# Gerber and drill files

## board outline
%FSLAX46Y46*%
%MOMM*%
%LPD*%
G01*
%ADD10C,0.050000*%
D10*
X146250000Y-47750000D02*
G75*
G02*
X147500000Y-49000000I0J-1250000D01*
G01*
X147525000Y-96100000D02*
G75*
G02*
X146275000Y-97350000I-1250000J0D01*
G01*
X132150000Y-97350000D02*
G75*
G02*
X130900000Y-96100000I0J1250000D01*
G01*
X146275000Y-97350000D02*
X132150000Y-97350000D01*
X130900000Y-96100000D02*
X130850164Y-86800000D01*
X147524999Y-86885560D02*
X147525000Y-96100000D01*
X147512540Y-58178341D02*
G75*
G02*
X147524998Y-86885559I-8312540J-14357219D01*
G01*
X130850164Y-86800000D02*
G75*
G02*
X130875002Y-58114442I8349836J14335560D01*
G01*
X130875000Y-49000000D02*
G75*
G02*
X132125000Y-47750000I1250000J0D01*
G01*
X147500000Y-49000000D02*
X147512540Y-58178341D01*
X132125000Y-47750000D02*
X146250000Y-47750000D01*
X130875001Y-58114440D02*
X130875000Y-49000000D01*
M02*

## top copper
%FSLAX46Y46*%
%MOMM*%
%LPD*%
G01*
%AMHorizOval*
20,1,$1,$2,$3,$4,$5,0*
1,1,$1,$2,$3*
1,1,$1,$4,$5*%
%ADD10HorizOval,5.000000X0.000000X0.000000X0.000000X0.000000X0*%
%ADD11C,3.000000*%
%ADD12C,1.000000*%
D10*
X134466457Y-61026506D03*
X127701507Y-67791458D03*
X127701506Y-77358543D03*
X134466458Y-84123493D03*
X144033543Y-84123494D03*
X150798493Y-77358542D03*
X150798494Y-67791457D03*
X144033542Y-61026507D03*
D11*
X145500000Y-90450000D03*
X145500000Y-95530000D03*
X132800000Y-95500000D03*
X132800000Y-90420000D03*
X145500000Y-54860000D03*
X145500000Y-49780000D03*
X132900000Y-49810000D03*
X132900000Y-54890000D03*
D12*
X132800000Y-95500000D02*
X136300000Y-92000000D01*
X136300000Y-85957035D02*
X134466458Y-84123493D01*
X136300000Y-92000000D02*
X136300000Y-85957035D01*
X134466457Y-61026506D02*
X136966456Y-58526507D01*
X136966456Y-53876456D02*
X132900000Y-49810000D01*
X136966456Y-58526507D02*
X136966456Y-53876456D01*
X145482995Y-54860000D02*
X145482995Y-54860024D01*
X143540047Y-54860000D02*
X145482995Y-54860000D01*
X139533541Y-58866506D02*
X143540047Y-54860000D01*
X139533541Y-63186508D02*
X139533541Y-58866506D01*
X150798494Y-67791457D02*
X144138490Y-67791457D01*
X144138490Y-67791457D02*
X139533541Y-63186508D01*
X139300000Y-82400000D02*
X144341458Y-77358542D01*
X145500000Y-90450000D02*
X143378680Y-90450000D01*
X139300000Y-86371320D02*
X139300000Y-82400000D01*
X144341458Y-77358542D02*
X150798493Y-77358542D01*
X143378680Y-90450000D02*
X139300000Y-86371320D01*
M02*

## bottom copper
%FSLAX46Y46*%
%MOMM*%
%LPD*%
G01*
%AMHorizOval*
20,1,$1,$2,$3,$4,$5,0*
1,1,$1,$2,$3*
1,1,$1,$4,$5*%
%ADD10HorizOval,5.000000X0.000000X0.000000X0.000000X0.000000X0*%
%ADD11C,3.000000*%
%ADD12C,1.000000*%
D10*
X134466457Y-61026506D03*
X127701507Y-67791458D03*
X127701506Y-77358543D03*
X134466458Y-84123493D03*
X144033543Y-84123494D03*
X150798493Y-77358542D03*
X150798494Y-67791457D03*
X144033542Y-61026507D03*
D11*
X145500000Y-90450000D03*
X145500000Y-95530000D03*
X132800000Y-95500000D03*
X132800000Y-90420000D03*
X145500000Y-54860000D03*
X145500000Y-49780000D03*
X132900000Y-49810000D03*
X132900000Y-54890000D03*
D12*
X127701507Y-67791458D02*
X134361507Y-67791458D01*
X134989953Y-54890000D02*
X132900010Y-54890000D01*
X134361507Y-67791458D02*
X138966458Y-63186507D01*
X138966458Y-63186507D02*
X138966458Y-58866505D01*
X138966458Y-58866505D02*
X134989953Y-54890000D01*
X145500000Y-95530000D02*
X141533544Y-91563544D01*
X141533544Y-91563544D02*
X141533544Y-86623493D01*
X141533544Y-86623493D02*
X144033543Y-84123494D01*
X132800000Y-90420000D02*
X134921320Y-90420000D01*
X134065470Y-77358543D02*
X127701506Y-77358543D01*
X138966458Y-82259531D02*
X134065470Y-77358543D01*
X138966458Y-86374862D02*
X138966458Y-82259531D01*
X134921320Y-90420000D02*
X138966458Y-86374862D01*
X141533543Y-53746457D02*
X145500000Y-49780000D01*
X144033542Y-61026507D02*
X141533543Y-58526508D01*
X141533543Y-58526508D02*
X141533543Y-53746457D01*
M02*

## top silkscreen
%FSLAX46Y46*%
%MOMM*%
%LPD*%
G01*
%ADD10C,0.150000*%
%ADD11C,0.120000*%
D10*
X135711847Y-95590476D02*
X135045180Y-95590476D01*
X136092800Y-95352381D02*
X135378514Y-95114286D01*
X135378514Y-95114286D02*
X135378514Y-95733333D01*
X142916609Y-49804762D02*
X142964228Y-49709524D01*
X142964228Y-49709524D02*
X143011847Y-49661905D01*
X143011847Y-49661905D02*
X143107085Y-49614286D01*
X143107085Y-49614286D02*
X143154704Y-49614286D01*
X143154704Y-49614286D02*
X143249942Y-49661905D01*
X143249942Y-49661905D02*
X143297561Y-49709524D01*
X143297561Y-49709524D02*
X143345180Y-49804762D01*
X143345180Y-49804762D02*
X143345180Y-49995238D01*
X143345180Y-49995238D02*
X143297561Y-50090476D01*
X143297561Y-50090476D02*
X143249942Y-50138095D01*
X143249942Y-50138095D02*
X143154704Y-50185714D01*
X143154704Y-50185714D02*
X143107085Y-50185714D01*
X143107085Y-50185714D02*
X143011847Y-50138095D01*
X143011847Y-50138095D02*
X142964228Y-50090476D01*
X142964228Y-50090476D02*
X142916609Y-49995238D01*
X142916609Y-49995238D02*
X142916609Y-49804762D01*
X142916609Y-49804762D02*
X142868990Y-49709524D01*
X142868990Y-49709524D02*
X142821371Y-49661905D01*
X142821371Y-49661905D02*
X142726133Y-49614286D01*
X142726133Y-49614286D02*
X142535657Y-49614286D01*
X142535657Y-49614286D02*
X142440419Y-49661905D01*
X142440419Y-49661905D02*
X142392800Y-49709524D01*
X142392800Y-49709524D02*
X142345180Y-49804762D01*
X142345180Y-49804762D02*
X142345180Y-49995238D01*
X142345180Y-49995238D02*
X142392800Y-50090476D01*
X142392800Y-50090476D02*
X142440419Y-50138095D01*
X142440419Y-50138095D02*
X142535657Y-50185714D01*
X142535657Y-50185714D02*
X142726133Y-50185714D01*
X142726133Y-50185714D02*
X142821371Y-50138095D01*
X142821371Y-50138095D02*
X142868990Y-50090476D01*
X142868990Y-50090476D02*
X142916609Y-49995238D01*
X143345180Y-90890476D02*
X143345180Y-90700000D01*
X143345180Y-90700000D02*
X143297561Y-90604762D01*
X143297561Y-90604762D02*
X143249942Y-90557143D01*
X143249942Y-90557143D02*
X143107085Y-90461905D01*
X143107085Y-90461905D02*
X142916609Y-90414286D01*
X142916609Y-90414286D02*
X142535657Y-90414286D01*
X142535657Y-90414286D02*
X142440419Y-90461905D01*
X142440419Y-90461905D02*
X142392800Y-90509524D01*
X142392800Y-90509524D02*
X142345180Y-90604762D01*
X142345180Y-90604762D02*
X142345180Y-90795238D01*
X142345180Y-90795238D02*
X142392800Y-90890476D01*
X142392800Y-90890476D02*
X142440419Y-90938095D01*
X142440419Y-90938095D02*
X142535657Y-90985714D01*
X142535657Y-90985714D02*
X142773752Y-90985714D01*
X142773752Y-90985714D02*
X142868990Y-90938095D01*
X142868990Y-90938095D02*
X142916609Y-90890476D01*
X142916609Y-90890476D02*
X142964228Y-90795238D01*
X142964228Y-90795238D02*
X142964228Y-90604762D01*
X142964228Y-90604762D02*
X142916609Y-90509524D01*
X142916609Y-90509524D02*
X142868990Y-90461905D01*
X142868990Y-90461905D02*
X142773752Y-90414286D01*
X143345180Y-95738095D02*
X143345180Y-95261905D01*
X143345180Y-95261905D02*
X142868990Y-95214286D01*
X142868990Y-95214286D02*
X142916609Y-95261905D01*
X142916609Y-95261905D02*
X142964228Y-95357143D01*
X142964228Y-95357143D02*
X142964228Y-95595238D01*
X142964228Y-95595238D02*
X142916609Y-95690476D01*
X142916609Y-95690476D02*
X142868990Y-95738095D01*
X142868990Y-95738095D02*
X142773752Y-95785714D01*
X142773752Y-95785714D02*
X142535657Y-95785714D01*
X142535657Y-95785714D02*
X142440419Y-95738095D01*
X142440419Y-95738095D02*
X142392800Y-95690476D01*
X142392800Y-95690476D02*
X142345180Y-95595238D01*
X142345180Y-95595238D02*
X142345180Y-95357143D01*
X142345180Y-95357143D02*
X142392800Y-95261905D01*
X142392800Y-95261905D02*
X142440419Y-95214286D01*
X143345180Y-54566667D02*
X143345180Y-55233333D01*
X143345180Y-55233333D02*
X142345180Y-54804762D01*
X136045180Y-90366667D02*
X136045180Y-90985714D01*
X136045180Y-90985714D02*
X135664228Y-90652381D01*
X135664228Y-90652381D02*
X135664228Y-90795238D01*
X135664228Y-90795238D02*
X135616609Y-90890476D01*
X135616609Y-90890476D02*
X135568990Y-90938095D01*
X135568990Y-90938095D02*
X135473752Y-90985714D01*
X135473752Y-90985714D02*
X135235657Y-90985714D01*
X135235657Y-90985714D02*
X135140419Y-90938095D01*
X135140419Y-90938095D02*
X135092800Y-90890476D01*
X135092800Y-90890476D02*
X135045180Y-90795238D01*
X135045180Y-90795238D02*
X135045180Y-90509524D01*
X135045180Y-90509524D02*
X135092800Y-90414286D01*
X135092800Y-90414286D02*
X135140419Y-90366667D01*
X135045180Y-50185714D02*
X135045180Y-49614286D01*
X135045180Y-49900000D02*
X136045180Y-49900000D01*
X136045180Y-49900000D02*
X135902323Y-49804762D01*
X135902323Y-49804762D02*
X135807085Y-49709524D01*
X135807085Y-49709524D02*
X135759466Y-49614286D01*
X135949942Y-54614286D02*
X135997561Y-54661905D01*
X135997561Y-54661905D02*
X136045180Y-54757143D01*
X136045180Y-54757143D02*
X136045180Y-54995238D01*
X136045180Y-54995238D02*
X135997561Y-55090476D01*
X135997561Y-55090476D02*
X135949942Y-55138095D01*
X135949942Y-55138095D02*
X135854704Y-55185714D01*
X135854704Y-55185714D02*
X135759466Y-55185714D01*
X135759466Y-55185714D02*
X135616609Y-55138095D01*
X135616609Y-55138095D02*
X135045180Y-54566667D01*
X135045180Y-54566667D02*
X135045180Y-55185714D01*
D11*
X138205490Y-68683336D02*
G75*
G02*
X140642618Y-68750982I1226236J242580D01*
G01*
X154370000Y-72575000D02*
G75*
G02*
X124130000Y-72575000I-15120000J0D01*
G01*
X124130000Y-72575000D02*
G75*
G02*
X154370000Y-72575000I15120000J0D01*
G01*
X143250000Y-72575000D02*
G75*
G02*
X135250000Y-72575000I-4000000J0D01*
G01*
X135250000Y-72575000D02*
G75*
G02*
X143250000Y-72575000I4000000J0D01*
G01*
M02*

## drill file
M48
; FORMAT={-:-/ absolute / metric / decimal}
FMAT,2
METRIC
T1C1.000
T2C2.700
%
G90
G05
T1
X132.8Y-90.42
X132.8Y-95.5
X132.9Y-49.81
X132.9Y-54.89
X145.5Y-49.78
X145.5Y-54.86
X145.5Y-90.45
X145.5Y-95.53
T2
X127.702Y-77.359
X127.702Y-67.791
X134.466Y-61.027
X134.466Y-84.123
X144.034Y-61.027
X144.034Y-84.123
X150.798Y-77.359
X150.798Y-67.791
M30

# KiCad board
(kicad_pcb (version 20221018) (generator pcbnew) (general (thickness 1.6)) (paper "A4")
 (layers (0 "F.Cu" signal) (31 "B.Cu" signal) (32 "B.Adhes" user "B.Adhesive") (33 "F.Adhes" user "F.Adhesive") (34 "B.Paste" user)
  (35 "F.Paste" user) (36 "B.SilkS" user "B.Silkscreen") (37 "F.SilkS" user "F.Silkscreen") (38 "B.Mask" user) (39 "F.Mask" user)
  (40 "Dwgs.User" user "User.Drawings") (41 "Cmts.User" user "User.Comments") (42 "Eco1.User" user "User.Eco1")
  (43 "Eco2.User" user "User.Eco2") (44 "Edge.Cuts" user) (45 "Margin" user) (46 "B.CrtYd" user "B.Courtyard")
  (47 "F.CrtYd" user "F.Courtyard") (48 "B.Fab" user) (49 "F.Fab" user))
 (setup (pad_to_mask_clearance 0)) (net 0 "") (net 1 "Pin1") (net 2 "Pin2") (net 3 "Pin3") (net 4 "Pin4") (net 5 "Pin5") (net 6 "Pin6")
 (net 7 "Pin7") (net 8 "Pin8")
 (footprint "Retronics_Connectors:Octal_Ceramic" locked (layer "F.Cu") (at 139.25 72.575 22.5)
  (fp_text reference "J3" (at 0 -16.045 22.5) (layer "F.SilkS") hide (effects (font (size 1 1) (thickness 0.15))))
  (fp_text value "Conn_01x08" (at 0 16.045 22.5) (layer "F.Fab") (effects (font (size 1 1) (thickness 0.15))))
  (fp_arc (start 0.524274 -3.995145) (mid 2.260212 -4.891133) (end 2.75 -3) (stroke (width 0.12) (type solid)) (layer "F.SilkS"))
  (fp_circle (center 0 0) (end 0 15.12) (stroke (width 0.12) (type solid)) (fill none) (layer "F.SilkS"))
  (fp_circle (center 0 0) (end 4 0) (stroke (width 0.12) (type solid)) (fill none) (layer "F.SilkS"))
  (pad "1" thru_hole oval locked (at 0 -12.5 22.5) (size 5 5) (drill 2.7) (layers "*.Cu" "*.Mask") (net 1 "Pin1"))
  (pad "2" thru_hole oval locked (at -8.838834 -8.838834 22.5) (size 5 5) (drill 2.7) (layers "*.Cu" "*.Mask") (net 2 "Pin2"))
  (pad "3" thru_hole oval locked (at -12.5 0 22.5) (size 5 5) (drill 2.7) (layers "*.Cu" "*.Mask") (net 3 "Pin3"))
  (pad "4" thru_hole oval locked (at -8.838834 8.838834 22.5) (size 5 5) (drill 2.7) (layers "*.Cu" "*.Mask") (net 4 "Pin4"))
  (pad "5" thru_hole oval locked (at 0 12.5 22.5) (size 5 5) (drill 2.7) (layers "*.Cu" "*.Mask") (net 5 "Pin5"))
  (pad "6" thru_hole oval locked (at 8.838834 8.838834 22.5) (size 5 5) (drill 2.7) (layers "*.Cu" "*.Mask") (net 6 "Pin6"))
  (pad "7" thru_hole oval locked (at 12.5 0 22.5) (size 5 5) (drill 2.7) (layers "*.Cu" "*.Mask") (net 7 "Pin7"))
  (pad "8" thru_hole oval locked (at 8.838834 -8.838834 22.5) (size 5 5) (drill 2.7) (layers "*.Cu" "*.Mask") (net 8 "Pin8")))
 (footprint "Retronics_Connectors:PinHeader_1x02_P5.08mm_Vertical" (layer "B.Cu") (at 145.5 90.45 180)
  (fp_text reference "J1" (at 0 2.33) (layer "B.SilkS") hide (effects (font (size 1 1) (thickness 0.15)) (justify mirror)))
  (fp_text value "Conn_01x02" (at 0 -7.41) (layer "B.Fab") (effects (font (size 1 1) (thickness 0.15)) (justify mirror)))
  (pad "1" thru_hole circle (at 0 0 180) (size 3 3) (drill 1) (layers "*.Cu" "*.Mask") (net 6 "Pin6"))
  (pad "2" thru_hole circle (at 0 -5.08 180) (size 3 3) (drill 1) (layers "*.Cu" "*.Mask") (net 5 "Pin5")))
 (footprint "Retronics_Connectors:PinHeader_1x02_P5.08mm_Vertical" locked (layer "B.Cu") (at 132.8 95.5)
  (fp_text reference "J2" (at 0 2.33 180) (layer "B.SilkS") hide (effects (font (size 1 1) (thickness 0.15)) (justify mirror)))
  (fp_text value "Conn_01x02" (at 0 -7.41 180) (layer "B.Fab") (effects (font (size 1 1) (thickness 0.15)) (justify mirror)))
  (pad "1" thru_hole circle locked (at 0 0) (size 3 3) (drill 1) (layers "*.Cu" "*.Mask") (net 4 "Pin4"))
  (pad "2" thru_hole circle locked (at 0 -5.08) (size 3 3) (drill 1) (layers "*.Cu" "*.Mask") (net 3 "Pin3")))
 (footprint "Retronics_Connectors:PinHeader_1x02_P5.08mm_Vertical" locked (layer "B.Cu") (at 145.5 54.86)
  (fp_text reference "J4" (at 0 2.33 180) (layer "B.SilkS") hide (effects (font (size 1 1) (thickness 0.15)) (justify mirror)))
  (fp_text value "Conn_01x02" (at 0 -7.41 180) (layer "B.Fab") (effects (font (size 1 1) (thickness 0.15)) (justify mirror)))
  (pad "1" thru_hole circle locked (at 0 0) (size 3 3) (drill 1) (layers "*.Cu" "*.Mask") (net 7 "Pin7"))
  (pad "2" thru_hole circle locked (at 0 -5.08) (size 3 3) (drill 1) (layers "*.Cu" "*.Mask") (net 8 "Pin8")))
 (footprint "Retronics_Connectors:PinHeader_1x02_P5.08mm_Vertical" (layer "B.Cu") (at 132.9 49.81 180)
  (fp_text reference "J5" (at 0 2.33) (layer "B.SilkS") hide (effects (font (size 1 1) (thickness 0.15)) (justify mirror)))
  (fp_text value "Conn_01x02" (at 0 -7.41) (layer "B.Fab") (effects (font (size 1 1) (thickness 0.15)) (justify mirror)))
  (pad "1" thru_hole circle (at 0 0 180) (size 3 3) (drill 1) (layers "*.Cu" "*.Mask") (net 1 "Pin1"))
  (pad "2" thru_hole circle (at 0 -5.08 180) (size 3 3) (drill 1) (layers "*.Cu" "*.Mask") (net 2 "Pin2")))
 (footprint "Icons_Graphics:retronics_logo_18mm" (layer "B.Cu") (at 142.3 72.536435 90)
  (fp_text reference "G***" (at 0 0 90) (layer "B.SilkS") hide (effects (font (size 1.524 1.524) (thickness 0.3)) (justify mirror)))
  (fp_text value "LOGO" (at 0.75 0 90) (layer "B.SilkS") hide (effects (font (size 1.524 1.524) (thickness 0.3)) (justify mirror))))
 (gr_arc (start 146.25 47.75) (mid 147.133883 48.116117) (end 147.5 49) (stroke (width 0.05) (type solid)) (layer "Edge.Cuts"))
 (gr_arc (start 147.525 96.1) (mid 147.158883 96.983883) (end 146.275 97.35) (stroke (width 0.05) (type solid)) (layer "Edge.Cuts"))
 (gr_arc (start 132.15 97.35) (mid 131.266117 96.983883) (end 130.9 96.1) (stroke (width 0.05) (type solid)) (layer "Edge.Cuts"))
 (gr_line (start 146.275 97.35) (end 132.15 97.35) (stroke (width 0.05) (type solid)) (layer "Edge.Cuts"))
 (gr_line (start 130.9 96.1) (end 130.850164 86.8) (stroke (width 0.05) (type solid)) (layer "Edge.Cuts"))
 (gr_line (start 147.524999 86.88556) (end 147.525 96.1) (stroke (width 0.05) (type solid)) (layer "Edge.Cuts"))
 (gr_arc (start 147.51254 58.178341) (mid 155.789998 72.528361) (end 147.524999 86.88556) (stroke (width 0.05) (type solid))
  (layer "Edge.Cuts"))
 (gr_arc (start 130.850164 86.8) (mid 122.610007 72.450075) (end 130.875001 58.11444) (stroke (width 0.05) (type solid)) (layer "Edge.Cuts"))
 (gr_arc (start 130.875 49) (mid 131.241117 48.116117) (end 132.125 47.75) (stroke (width 0.05) (type solid)) (layer "Edge.Cuts"))
 (gr_line (start 147.5 49) (end 147.51254 58.178341) (stroke (width 0.05) (type solid)) (layer "Edge.Cuts"))
 (gr_line (start 132.125 47.75) (end 146.25 47.75) (stroke (width 0.05) (type solid)) (layer "Edge.Cuts"))
 (gr_line (start 130.875001 58.11444) (end 130.875 49) (stroke (width 0.05) (type solid)) (layer "Edge.Cuts"))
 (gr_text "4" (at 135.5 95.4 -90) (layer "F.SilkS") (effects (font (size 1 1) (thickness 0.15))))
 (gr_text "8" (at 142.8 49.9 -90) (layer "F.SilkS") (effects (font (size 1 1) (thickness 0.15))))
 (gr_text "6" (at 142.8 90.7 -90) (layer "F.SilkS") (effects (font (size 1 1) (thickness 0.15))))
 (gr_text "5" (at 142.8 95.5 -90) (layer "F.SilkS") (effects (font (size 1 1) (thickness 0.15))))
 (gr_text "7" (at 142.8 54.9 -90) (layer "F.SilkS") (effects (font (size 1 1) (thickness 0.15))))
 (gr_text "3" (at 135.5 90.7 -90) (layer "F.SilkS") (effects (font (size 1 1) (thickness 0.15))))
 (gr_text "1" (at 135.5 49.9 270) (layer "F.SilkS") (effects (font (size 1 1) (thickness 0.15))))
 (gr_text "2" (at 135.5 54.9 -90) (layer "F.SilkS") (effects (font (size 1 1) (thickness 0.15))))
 (segment (start 127.701507 67.791458) (end 134.361507 67.791458) (width 1) (layer "B.Cu") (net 2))
 (segment (start 134.989953 54.89) (end 132.90001 54.89) (width 1) (layer "B.Cu") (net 2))
 (segment (start 134.361507 67.791458) (end 138.966458 63.186507) (width 1) (layer "B.Cu") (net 2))
 (segment (start 138.966458 63.186507) (end 138.966458 58.866505) (width 1) (layer "B.Cu") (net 2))
 (segment (start 138.966458 58.866505) (end 134.989953 54.89) (width 1) (layer "B.Cu") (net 2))
 (segment (start 145.5 95.53) (end 141.533544 91.563544) (width 1) (layer "B.Cu") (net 5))
 (segment (start 141.533544 91.563544) (end 141.533544 86.623493) (width 1) (layer "B.Cu") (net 5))
 (segment (start 141.533544 86.623493) (end 144.033543 84.123494) (width 1) (layer "B.Cu") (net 5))
 (segment (start 132.8 90.42) (end 134.92132 90.42) (width 1) (layer "B.Cu") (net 3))
 (segment (start 134.06547 77.358543) (end 127.701506 77.358543) (width 1) (layer "B.Cu") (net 3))
 (segment (start 138.966458 82.259531) (end 134.06547 77.358543) (width 1) (layer "B.Cu") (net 3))
 (segment (start 138.966458 86.374862) (end 138.966458 82.259531) (width 1) (layer "B.Cu") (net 3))
 (segment (start 134.92132 90.42) (end 138.966458 86.374862) (width 1) (layer "B.Cu") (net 3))
 (segment (start 132.8 95.5) (end 136.3 92) (width 1) (layer "F.Cu") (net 4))
 (segment (start 136.3 85.957035) (end 134.466458 84.123493) (width 1) (layer "F.Cu") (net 4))
 (segment (start 136.3 92) (end 136.3 85.957035) (width 1) (layer "F.Cu") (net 4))
 (segment (start 134.466457 61.026506) (end 136.966456 58.526507) (width 1) (layer "F.Cu") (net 1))
 (segment (start 136.966456 53.876456) (end 132.9 49.81) (width 1) (layer "F.Cu") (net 1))
 (segment (start 136.966456 58.526507) (end 136.966456 53.876456) (width 1) (layer "F.Cu") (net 1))
 (segment (start 141.533543 53.746457) (end 145.5 49.78) (width 1) (layer "B.Cu") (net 8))
 (segment (start 144.033542 61.026507) (end 141.533543 58.526508) (width 1) (layer "B.Cu") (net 8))
 (segment (start 141.533543 58.526508) (end 141.533543 53.746457) (width 1) (layer "B.Cu") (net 8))
 (segment (start 145.482995 54.86) (end 145.482995 54.860024) (width 1) (layer "F.Cu") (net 7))
 (segment (start 143.540047 54.86) (end 145.482995 54.86) (width 1) (layer "F.Cu") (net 7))
 (segment (start 139.533541 58.866506) (end 143.540047 54.86) (width 1) (layer "F.Cu") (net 7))
 (segment (start 139.533541 63.186508) (end 139.533541 58.866506) (width 1) (layer "F.Cu") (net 7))
 (segment (start 150.798494 67.791457) (end 144.13849 67.791457) (width 1) (layer "F.Cu") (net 7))
 (segment (start 144.13849 67.791457) (end 139.533541 63.186508) (width 1) (layer "F.Cu") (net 7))
 (segment (start 139.3 82.4) (end 144.341458 77.358542) (width 1) (layer "F.Cu") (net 6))
 (segment (start 145.5 90.45) (end 143.37868 90.45) (width 1) (layer "F.Cu") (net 6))
 (segment (start 139.3 86.37132) (end 139.3 82.4) (width 1) (layer "F.Cu") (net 6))
 (segment (start 144.341458 77.358542) (end 150.798493 77.358542) (width 1) (layer "F.Cu") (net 6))
 (segment (start 143.37868 90.45) (end 139.3 86.37132) (width 1) (layer "F.Cu") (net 6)))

